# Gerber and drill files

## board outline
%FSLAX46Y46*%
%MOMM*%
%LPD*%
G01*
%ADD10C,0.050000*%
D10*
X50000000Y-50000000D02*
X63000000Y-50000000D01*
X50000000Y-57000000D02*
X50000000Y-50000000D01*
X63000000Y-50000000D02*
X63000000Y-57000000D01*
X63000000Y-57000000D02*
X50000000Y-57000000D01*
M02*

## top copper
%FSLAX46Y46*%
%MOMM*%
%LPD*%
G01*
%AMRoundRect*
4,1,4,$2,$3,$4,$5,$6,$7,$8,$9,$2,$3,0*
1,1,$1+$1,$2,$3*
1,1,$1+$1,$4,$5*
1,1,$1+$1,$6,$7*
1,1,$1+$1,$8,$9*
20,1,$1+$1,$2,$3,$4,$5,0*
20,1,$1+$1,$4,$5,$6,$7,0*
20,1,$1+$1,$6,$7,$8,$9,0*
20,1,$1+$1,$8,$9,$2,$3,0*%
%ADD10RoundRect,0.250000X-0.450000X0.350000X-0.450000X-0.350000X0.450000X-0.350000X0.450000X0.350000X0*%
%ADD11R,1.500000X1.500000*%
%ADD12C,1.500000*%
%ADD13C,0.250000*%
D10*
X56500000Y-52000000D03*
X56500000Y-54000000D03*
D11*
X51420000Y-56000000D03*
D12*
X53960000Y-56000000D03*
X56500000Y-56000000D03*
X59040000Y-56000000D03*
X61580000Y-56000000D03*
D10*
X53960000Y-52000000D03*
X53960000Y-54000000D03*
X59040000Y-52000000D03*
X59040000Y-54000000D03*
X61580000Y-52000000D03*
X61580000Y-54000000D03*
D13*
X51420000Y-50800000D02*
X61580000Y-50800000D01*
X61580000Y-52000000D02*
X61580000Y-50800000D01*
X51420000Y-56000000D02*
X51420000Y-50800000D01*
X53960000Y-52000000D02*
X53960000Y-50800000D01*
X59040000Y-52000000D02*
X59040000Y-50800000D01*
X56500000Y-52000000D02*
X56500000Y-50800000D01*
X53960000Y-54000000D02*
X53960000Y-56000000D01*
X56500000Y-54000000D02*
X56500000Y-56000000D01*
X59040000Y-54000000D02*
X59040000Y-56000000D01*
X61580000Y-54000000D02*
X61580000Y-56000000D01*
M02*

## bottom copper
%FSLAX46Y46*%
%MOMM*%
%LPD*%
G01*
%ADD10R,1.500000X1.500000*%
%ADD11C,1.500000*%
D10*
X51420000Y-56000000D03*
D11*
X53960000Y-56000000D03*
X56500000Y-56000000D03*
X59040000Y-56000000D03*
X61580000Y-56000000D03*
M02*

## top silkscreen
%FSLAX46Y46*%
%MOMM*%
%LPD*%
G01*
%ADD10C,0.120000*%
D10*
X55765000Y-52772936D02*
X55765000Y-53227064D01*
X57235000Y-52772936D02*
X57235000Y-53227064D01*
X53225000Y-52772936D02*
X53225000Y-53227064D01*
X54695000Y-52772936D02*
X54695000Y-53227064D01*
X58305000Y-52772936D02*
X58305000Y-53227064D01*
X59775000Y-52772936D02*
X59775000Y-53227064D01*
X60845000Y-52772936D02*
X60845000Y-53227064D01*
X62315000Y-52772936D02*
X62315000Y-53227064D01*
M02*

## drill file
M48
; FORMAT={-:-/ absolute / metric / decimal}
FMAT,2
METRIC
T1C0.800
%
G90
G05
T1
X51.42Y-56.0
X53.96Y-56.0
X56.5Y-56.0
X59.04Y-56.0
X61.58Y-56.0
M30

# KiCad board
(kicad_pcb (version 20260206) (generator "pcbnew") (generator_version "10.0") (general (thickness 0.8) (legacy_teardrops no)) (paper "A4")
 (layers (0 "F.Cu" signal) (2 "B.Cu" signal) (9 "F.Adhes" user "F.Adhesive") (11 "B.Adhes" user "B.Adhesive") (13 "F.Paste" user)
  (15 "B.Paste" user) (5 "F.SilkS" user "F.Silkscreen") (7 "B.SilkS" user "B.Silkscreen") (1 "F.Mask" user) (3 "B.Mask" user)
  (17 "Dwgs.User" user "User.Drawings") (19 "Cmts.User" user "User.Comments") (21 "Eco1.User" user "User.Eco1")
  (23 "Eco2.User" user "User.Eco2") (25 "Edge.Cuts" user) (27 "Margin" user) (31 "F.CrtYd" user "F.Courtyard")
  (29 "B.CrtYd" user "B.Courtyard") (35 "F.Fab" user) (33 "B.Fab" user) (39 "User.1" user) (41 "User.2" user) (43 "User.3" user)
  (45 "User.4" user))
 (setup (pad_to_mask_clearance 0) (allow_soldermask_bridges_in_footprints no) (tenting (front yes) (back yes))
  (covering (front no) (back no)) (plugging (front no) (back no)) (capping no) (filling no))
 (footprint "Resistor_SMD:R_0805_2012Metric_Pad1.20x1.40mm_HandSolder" (layer "F.Cu") (at 56.5 53 -90)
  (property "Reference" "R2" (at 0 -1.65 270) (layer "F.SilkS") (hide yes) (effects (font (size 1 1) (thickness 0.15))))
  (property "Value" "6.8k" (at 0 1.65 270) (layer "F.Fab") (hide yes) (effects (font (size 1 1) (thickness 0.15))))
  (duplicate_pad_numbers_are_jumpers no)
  (fp_line (start -0.227064 0.735) (end 0.227064 0.735) (stroke (width 0.12) (type solid)) (layer "F.SilkS"))
  (fp_line (start -0.227064 -0.735) (end 0.227064 -0.735) (stroke (width 0.12) (type solid)) (layer "F.SilkS"))
  (pad "1" smd roundrect (at -1 0 270) (size 1.2 1.4) (layers "F.Cu" "F.Mask" "F.Paste") (roundrect_rratio 0.208333) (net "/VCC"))
  (pad "2" smd roundrect (at 1 0 270) (size 1.2 1.4) (layers "F.Cu" "F.Mask" "F.Paste") (roundrect_rratio 0.208333) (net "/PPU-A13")))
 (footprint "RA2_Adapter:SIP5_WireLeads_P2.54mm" (layer "F.Cu") (at 51.42 56)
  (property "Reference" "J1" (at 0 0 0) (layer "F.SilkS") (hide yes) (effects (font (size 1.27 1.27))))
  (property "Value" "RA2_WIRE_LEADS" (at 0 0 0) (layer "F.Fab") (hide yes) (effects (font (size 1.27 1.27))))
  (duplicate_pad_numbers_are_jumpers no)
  (pad "1" thru_hole rect (at 0 0) (size 1.5 1.5) (drill 0.8) (layers "*.Cu" "*.Mask") (remove_unused_layers no) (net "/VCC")
   (thermal_bridge_angle 45))
  (pad "2" thru_hole circle (at 2.54 0) (size 1.5 1.5) (drill 0.8) (layers "*.Cu" "*.Mask") (remove_unused_layers no) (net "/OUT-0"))
  (pad "3" thru_hole circle (at 5.08 0) (size 1.5 1.5) (drill 0.8) (layers "*.Cu" "*.Mask") (remove_unused_layers no) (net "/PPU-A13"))
  (pad "4" thru_hole circle (at 7.62 0) (size 1.5 1.5) (drill 0.8) (layers "*.Cu" "*.Mask") (remove_unused_layers no) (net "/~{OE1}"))
  (pad "5" thru_hole circle (at 10.16 0) (size 1.5 1.5) (drill 0.8) (layers "*.Cu" "*.Mask") (remove_unused_layers no) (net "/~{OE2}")))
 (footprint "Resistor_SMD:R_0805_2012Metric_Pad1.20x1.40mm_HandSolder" (layer "F.Cu") (at 53.96 53 -90)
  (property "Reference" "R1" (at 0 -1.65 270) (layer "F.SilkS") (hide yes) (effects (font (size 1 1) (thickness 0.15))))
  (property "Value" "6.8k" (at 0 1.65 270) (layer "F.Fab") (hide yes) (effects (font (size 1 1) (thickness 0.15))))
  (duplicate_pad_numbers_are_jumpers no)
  (fp_line (start -0.227064 0.735) (end 0.227064 0.735) (stroke (width 0.12) (type solid)) (layer "F.SilkS"))
  (fp_line (start -0.227064 -0.735) (end 0.227064 -0.735) (stroke (width 0.12) (type solid)) (layer "F.SilkS"))
  (pad "1" smd roundrect (at -1 0 270) (size 1.2 1.4) (layers "F.Cu" "F.Mask" "F.Paste") (roundrect_rratio 0.208333) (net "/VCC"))
  (pad "2" smd roundrect (at 1 0 270) (size 1.2 1.4) (layers "F.Cu" "F.Mask" "F.Paste") (roundrect_rratio 0.208333) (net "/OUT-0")))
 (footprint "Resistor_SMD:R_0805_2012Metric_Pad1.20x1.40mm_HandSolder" (layer "F.Cu") (at 59.04 53 -90)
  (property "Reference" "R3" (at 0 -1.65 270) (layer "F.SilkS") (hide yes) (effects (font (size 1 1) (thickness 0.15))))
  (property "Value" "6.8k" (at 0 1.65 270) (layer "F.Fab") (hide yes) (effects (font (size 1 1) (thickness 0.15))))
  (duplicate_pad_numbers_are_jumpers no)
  (fp_line (start -0.227064 0.735) (end 0.227064 0.735) (stroke (width 0.12) (type solid)) (layer "F.SilkS"))
  (fp_line (start -0.227064 -0.735) (end 0.227064 -0.735) (stroke (width 0.12) (type solid)) (layer "F.SilkS"))
  (pad "1" smd roundrect (at -1 0 270) (size 1.2 1.4) (layers "F.Cu" "F.Mask" "F.Paste") (roundrect_rratio 0.208333) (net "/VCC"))
  (pad "2" smd roundrect (at 1 0 270) (size 1.2 1.4) (layers "F.Cu" "F.Mask" "F.Paste") (roundrect_rratio 0.208333) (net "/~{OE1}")))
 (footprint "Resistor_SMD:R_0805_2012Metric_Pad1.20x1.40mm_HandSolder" (layer "F.Cu") (at 61.58 53 -90)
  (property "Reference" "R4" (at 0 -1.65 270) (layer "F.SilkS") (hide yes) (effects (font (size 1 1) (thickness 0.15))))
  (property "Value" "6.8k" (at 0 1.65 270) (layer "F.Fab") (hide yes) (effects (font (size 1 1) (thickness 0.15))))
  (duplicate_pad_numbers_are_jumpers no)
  (fp_line (start -0.227064 0.735) (end 0.227064 0.735) (stroke (width 0.12) (type solid)) (layer "F.SilkS"))
  (fp_line (start -0.227064 -0.735) (end 0.227064 -0.735) (stroke (width 0.12) (type solid)) (layer "F.SilkS"))
  (pad "1" smd roundrect (at -1 0 270) (size 1.2 1.4) (layers "F.Cu" "F.Mask" "F.Paste") (roundrect_rratio 0.208333) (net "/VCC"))
  (pad "2" smd roundrect (at 1 0 270) (size 1.2 1.4) (layers "F.Cu" "F.Mask" "F.Paste") (roundrect_rratio 0.208333) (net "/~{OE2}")))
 (gr_line (start 50 50) (end 63 50) (stroke (width 0.05) (type default)) (layer "Edge.Cuts"))
 (gr_line (start 50 57) (end 50 50) (stroke (width 0.05) (type default)) (layer "Edge.Cuts"))
 (gr_line (start 63 50) (end 63 57) (stroke (width 0.05) (type default)) (layer "Edge.Cuts"))
 (gr_line (start 63 57) (end 50 57) (stroke (width 0.05) (type default)) (layer "Edge.Cuts"))
 (segment (start 51.42 50.8) (end 61.58 50.8) (width 0.25) (layer "F.Cu") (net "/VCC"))
 (segment (start 61.58 52) (end 61.58 50.8) (width 0.25) (layer "F.Cu") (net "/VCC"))
 (segment (start 51.42 56) (end 51.42 50.8) (width 0.25) (layer "F.Cu") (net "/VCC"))
 (segment (start 53.96 52) (end 53.96 50.8) (width 0.25) (layer "F.Cu") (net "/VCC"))
 (segment (start 59.04 52) (end 59.04 50.8) (width 0.25) (layer "F.Cu") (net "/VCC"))
 (segment (start 56.5 52) (end 56.5 50.8) (width 0.25) (layer "F.Cu") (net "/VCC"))
 (segment (start 53.96 54) (end 53.96 56) (width 0.25) (layer "F.Cu") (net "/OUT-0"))
 (segment (start 56.5 54) (end 56.5 56) (width 0.25) (layer "F.Cu") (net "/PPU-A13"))
 (segment (start 59.04 54) (end 59.04 56) (width 0.25) (layer "F.Cu") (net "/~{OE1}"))
 (segment (start 61.58 54) (end 61.58 56) (width 0.25) (layer "F.Cu") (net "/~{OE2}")))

